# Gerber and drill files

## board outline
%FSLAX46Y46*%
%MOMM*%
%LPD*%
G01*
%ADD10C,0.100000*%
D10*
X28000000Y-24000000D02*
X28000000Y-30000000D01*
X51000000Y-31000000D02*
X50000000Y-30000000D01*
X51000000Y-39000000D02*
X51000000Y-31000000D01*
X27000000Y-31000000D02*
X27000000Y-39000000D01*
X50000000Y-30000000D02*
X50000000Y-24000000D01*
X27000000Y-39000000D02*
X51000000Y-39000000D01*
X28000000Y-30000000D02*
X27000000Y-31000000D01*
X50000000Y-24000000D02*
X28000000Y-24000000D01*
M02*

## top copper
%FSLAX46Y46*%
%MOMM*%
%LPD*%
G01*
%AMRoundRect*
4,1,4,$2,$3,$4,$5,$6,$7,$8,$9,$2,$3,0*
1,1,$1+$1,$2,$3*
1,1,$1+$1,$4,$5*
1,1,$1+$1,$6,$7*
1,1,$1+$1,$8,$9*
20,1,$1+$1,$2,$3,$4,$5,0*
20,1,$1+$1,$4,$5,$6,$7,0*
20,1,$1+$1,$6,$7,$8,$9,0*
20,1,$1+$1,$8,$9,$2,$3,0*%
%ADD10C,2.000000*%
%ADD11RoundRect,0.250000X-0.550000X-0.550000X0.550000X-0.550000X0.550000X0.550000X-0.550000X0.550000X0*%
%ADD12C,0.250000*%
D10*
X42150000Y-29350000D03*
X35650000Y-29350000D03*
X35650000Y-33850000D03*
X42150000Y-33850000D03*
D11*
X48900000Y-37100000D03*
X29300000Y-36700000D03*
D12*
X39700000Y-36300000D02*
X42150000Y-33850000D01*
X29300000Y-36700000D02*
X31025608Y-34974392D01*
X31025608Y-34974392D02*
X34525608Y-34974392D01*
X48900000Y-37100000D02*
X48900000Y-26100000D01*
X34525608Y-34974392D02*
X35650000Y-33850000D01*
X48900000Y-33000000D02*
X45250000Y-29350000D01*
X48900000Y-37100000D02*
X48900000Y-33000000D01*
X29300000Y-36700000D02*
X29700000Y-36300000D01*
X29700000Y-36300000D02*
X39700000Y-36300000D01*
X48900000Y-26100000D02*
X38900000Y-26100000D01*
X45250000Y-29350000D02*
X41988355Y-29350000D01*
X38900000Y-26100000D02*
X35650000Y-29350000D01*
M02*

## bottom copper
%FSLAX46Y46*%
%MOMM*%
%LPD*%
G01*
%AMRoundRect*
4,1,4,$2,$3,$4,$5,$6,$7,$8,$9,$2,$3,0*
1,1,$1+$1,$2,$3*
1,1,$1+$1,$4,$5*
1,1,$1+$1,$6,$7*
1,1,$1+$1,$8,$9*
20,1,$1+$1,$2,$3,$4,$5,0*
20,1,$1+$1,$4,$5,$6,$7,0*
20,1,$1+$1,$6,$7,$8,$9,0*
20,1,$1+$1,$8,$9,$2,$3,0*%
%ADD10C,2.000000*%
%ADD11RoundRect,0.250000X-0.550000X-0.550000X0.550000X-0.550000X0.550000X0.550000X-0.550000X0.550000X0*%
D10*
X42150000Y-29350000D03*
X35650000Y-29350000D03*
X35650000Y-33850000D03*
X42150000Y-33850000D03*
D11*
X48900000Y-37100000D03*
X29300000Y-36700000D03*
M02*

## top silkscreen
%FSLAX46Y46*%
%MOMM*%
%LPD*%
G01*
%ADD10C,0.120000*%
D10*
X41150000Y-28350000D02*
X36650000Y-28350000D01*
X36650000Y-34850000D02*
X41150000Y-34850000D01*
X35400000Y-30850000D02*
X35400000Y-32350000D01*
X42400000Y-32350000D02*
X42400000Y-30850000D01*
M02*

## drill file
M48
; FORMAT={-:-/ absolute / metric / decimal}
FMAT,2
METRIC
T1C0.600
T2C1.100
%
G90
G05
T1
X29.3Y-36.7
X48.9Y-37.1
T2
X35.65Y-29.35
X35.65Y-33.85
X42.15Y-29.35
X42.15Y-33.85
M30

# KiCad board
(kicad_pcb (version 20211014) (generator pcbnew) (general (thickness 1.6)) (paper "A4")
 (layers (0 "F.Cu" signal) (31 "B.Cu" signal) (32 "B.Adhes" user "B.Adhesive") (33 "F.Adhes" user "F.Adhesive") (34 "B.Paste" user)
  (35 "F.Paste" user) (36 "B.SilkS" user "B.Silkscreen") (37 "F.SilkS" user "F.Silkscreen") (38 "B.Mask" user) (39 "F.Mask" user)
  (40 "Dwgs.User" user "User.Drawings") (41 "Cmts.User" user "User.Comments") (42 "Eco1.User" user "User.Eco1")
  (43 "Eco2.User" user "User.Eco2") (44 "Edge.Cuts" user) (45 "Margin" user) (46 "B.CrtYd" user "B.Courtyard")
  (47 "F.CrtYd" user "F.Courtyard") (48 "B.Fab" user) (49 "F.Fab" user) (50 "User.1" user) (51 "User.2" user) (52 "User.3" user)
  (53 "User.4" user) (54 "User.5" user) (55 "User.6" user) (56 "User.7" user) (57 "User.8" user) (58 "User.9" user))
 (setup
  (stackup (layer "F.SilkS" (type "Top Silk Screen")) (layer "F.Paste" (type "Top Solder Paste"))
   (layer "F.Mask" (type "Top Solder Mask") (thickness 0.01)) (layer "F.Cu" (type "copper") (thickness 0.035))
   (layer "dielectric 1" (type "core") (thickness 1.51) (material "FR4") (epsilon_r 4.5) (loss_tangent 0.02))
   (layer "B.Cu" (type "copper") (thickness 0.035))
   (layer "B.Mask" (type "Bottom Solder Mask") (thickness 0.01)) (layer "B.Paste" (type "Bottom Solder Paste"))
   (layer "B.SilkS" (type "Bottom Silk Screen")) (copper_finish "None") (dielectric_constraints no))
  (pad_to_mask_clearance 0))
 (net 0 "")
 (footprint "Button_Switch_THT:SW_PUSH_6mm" (layer "F.Cu") (at 35.65 29.35)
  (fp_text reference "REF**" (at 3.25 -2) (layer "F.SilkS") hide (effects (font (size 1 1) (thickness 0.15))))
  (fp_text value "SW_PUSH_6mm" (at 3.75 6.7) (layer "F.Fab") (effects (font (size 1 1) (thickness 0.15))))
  (fp_line (start 5.5 -1) (end 1 -1) (layer "F.SilkS") (width 0.12))
  (fp_line (start 1 5.5) (end 5.5 5.5) (layer "F.SilkS") (width 0.12))
  (fp_line (start -0.25 1.5) (end -0.25 3) (layer "F.SilkS") (width 0.12))
  (fp_line (start 6.75 3) (end 6.75 1.5) (layer "F.SilkS") (width 0.12))
  (pad "1" thru_hole circle (at 6.5 0 90) (size 2 2) (drill 1.1) (layers *.Cu *.Mask))
  (pad "1" thru_hole circle (at 0 0 90) (size 2 2) (drill 1.1) (layers *.Cu *.Mask))
  (pad "2" thru_hole circle (at 0 4.5 90) (size 2 2) (drill 1.1) (layers *.Cu *.Mask))
  (pad "2" thru_hole circle (at 6.5 4.5 90) (size 2 2) (drill 1.1) (layers *.Cu *.Mask)))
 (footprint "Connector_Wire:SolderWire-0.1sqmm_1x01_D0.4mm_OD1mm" (layer "F.Cu") (at 48.9 37.1)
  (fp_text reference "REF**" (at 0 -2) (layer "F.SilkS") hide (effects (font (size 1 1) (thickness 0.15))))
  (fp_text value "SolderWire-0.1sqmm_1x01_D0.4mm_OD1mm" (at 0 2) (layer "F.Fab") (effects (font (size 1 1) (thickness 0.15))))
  (pad "1" thru_hole roundrect (at 0 0) (size 1.6 1.6) (drill 0.6) (layers *.Cu *.Mask) (roundrect_rratio 0.15625)))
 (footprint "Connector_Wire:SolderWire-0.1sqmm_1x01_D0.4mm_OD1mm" (layer "F.Cu") (at 29.3 36.7)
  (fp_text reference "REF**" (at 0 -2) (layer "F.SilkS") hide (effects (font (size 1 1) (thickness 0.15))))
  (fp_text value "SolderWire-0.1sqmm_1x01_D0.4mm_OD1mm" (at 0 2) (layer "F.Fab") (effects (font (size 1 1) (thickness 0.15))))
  (pad "1" thru_hole roundrect (at 0 0) (size 1.6 1.6) (drill 0.6) (layers *.Cu *.Mask) (roundrect_rratio 0.15625)))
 (gr_line (start 28 24) (end 28 30) (layer "Edge.Cuts") (width 0.1))
 (gr_line (start 51 31) (end 50 30) (layer "Edge.Cuts") (width 0.1))
 (gr_line (start 51 39) (end 51 31) (layer "Edge.Cuts") (width 0.1))
 (gr_line (start 27 31) (end 27 39) (layer "Edge.Cuts") (width 0.1))
 (gr_line (start 50 30) (end 50 24) (layer "Edge.Cuts") (width 0.1))
 (gr_line (start 27 39) (end 51 39) (layer "Edge.Cuts") (width 0.1))
 (gr_line (start 28 30) (end 27 31) (layer "Edge.Cuts") (width 0.1))
 (gr_line (start 50 24) (end 28 24) (layer "Edge.Cuts") (width 0.1))
 (segment (start 39.7 36.3) (end 42.15 33.85) (width 0.25) (layer "F.Cu") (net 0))
 (segment (start 29.3 36.7) (end 31.025608 34.974392) (width 0.25) (layer "F.Cu") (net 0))
 (segment (start 31.025608 34.974392) (end 34.525608 34.974392) (width 0.25) (layer "F.Cu") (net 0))
 (segment (start 48.9 37.1) (end 48.9 26.1) (width 0.25) (layer "F.Cu") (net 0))
 (segment (start 34.525608 34.974392) (end 35.65 33.85) (width 0.25) (layer "F.Cu") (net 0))
 (segment (start 48.9 33) (end 45.25 29.35) (width 0.25) (layer "F.Cu") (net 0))
 (segment (start 48.9 37.1) (end 48.9 33) (width 0.25) (layer "F.Cu") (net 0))
 (segment (start 29.3 36.7) (end 29.7 36.3) (width 0.25) (layer "F.Cu") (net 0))
 (segment (start 29.7 36.3) (end 39.7 36.3) (width 0.25) (layer "F.Cu") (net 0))
 (segment (start 48.9 26.1) (end 38.9 26.1) (width 0.25) (layer "F.Cu") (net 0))
 (segment (start 45.25 29.35) (end 41.988355 29.35) (width 0.25) (layer "F.Cu") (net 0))
 (segment (start 38.9 26.1) (end 35.65 29.35) (width 0.25) (layer "F.Cu") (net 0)))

